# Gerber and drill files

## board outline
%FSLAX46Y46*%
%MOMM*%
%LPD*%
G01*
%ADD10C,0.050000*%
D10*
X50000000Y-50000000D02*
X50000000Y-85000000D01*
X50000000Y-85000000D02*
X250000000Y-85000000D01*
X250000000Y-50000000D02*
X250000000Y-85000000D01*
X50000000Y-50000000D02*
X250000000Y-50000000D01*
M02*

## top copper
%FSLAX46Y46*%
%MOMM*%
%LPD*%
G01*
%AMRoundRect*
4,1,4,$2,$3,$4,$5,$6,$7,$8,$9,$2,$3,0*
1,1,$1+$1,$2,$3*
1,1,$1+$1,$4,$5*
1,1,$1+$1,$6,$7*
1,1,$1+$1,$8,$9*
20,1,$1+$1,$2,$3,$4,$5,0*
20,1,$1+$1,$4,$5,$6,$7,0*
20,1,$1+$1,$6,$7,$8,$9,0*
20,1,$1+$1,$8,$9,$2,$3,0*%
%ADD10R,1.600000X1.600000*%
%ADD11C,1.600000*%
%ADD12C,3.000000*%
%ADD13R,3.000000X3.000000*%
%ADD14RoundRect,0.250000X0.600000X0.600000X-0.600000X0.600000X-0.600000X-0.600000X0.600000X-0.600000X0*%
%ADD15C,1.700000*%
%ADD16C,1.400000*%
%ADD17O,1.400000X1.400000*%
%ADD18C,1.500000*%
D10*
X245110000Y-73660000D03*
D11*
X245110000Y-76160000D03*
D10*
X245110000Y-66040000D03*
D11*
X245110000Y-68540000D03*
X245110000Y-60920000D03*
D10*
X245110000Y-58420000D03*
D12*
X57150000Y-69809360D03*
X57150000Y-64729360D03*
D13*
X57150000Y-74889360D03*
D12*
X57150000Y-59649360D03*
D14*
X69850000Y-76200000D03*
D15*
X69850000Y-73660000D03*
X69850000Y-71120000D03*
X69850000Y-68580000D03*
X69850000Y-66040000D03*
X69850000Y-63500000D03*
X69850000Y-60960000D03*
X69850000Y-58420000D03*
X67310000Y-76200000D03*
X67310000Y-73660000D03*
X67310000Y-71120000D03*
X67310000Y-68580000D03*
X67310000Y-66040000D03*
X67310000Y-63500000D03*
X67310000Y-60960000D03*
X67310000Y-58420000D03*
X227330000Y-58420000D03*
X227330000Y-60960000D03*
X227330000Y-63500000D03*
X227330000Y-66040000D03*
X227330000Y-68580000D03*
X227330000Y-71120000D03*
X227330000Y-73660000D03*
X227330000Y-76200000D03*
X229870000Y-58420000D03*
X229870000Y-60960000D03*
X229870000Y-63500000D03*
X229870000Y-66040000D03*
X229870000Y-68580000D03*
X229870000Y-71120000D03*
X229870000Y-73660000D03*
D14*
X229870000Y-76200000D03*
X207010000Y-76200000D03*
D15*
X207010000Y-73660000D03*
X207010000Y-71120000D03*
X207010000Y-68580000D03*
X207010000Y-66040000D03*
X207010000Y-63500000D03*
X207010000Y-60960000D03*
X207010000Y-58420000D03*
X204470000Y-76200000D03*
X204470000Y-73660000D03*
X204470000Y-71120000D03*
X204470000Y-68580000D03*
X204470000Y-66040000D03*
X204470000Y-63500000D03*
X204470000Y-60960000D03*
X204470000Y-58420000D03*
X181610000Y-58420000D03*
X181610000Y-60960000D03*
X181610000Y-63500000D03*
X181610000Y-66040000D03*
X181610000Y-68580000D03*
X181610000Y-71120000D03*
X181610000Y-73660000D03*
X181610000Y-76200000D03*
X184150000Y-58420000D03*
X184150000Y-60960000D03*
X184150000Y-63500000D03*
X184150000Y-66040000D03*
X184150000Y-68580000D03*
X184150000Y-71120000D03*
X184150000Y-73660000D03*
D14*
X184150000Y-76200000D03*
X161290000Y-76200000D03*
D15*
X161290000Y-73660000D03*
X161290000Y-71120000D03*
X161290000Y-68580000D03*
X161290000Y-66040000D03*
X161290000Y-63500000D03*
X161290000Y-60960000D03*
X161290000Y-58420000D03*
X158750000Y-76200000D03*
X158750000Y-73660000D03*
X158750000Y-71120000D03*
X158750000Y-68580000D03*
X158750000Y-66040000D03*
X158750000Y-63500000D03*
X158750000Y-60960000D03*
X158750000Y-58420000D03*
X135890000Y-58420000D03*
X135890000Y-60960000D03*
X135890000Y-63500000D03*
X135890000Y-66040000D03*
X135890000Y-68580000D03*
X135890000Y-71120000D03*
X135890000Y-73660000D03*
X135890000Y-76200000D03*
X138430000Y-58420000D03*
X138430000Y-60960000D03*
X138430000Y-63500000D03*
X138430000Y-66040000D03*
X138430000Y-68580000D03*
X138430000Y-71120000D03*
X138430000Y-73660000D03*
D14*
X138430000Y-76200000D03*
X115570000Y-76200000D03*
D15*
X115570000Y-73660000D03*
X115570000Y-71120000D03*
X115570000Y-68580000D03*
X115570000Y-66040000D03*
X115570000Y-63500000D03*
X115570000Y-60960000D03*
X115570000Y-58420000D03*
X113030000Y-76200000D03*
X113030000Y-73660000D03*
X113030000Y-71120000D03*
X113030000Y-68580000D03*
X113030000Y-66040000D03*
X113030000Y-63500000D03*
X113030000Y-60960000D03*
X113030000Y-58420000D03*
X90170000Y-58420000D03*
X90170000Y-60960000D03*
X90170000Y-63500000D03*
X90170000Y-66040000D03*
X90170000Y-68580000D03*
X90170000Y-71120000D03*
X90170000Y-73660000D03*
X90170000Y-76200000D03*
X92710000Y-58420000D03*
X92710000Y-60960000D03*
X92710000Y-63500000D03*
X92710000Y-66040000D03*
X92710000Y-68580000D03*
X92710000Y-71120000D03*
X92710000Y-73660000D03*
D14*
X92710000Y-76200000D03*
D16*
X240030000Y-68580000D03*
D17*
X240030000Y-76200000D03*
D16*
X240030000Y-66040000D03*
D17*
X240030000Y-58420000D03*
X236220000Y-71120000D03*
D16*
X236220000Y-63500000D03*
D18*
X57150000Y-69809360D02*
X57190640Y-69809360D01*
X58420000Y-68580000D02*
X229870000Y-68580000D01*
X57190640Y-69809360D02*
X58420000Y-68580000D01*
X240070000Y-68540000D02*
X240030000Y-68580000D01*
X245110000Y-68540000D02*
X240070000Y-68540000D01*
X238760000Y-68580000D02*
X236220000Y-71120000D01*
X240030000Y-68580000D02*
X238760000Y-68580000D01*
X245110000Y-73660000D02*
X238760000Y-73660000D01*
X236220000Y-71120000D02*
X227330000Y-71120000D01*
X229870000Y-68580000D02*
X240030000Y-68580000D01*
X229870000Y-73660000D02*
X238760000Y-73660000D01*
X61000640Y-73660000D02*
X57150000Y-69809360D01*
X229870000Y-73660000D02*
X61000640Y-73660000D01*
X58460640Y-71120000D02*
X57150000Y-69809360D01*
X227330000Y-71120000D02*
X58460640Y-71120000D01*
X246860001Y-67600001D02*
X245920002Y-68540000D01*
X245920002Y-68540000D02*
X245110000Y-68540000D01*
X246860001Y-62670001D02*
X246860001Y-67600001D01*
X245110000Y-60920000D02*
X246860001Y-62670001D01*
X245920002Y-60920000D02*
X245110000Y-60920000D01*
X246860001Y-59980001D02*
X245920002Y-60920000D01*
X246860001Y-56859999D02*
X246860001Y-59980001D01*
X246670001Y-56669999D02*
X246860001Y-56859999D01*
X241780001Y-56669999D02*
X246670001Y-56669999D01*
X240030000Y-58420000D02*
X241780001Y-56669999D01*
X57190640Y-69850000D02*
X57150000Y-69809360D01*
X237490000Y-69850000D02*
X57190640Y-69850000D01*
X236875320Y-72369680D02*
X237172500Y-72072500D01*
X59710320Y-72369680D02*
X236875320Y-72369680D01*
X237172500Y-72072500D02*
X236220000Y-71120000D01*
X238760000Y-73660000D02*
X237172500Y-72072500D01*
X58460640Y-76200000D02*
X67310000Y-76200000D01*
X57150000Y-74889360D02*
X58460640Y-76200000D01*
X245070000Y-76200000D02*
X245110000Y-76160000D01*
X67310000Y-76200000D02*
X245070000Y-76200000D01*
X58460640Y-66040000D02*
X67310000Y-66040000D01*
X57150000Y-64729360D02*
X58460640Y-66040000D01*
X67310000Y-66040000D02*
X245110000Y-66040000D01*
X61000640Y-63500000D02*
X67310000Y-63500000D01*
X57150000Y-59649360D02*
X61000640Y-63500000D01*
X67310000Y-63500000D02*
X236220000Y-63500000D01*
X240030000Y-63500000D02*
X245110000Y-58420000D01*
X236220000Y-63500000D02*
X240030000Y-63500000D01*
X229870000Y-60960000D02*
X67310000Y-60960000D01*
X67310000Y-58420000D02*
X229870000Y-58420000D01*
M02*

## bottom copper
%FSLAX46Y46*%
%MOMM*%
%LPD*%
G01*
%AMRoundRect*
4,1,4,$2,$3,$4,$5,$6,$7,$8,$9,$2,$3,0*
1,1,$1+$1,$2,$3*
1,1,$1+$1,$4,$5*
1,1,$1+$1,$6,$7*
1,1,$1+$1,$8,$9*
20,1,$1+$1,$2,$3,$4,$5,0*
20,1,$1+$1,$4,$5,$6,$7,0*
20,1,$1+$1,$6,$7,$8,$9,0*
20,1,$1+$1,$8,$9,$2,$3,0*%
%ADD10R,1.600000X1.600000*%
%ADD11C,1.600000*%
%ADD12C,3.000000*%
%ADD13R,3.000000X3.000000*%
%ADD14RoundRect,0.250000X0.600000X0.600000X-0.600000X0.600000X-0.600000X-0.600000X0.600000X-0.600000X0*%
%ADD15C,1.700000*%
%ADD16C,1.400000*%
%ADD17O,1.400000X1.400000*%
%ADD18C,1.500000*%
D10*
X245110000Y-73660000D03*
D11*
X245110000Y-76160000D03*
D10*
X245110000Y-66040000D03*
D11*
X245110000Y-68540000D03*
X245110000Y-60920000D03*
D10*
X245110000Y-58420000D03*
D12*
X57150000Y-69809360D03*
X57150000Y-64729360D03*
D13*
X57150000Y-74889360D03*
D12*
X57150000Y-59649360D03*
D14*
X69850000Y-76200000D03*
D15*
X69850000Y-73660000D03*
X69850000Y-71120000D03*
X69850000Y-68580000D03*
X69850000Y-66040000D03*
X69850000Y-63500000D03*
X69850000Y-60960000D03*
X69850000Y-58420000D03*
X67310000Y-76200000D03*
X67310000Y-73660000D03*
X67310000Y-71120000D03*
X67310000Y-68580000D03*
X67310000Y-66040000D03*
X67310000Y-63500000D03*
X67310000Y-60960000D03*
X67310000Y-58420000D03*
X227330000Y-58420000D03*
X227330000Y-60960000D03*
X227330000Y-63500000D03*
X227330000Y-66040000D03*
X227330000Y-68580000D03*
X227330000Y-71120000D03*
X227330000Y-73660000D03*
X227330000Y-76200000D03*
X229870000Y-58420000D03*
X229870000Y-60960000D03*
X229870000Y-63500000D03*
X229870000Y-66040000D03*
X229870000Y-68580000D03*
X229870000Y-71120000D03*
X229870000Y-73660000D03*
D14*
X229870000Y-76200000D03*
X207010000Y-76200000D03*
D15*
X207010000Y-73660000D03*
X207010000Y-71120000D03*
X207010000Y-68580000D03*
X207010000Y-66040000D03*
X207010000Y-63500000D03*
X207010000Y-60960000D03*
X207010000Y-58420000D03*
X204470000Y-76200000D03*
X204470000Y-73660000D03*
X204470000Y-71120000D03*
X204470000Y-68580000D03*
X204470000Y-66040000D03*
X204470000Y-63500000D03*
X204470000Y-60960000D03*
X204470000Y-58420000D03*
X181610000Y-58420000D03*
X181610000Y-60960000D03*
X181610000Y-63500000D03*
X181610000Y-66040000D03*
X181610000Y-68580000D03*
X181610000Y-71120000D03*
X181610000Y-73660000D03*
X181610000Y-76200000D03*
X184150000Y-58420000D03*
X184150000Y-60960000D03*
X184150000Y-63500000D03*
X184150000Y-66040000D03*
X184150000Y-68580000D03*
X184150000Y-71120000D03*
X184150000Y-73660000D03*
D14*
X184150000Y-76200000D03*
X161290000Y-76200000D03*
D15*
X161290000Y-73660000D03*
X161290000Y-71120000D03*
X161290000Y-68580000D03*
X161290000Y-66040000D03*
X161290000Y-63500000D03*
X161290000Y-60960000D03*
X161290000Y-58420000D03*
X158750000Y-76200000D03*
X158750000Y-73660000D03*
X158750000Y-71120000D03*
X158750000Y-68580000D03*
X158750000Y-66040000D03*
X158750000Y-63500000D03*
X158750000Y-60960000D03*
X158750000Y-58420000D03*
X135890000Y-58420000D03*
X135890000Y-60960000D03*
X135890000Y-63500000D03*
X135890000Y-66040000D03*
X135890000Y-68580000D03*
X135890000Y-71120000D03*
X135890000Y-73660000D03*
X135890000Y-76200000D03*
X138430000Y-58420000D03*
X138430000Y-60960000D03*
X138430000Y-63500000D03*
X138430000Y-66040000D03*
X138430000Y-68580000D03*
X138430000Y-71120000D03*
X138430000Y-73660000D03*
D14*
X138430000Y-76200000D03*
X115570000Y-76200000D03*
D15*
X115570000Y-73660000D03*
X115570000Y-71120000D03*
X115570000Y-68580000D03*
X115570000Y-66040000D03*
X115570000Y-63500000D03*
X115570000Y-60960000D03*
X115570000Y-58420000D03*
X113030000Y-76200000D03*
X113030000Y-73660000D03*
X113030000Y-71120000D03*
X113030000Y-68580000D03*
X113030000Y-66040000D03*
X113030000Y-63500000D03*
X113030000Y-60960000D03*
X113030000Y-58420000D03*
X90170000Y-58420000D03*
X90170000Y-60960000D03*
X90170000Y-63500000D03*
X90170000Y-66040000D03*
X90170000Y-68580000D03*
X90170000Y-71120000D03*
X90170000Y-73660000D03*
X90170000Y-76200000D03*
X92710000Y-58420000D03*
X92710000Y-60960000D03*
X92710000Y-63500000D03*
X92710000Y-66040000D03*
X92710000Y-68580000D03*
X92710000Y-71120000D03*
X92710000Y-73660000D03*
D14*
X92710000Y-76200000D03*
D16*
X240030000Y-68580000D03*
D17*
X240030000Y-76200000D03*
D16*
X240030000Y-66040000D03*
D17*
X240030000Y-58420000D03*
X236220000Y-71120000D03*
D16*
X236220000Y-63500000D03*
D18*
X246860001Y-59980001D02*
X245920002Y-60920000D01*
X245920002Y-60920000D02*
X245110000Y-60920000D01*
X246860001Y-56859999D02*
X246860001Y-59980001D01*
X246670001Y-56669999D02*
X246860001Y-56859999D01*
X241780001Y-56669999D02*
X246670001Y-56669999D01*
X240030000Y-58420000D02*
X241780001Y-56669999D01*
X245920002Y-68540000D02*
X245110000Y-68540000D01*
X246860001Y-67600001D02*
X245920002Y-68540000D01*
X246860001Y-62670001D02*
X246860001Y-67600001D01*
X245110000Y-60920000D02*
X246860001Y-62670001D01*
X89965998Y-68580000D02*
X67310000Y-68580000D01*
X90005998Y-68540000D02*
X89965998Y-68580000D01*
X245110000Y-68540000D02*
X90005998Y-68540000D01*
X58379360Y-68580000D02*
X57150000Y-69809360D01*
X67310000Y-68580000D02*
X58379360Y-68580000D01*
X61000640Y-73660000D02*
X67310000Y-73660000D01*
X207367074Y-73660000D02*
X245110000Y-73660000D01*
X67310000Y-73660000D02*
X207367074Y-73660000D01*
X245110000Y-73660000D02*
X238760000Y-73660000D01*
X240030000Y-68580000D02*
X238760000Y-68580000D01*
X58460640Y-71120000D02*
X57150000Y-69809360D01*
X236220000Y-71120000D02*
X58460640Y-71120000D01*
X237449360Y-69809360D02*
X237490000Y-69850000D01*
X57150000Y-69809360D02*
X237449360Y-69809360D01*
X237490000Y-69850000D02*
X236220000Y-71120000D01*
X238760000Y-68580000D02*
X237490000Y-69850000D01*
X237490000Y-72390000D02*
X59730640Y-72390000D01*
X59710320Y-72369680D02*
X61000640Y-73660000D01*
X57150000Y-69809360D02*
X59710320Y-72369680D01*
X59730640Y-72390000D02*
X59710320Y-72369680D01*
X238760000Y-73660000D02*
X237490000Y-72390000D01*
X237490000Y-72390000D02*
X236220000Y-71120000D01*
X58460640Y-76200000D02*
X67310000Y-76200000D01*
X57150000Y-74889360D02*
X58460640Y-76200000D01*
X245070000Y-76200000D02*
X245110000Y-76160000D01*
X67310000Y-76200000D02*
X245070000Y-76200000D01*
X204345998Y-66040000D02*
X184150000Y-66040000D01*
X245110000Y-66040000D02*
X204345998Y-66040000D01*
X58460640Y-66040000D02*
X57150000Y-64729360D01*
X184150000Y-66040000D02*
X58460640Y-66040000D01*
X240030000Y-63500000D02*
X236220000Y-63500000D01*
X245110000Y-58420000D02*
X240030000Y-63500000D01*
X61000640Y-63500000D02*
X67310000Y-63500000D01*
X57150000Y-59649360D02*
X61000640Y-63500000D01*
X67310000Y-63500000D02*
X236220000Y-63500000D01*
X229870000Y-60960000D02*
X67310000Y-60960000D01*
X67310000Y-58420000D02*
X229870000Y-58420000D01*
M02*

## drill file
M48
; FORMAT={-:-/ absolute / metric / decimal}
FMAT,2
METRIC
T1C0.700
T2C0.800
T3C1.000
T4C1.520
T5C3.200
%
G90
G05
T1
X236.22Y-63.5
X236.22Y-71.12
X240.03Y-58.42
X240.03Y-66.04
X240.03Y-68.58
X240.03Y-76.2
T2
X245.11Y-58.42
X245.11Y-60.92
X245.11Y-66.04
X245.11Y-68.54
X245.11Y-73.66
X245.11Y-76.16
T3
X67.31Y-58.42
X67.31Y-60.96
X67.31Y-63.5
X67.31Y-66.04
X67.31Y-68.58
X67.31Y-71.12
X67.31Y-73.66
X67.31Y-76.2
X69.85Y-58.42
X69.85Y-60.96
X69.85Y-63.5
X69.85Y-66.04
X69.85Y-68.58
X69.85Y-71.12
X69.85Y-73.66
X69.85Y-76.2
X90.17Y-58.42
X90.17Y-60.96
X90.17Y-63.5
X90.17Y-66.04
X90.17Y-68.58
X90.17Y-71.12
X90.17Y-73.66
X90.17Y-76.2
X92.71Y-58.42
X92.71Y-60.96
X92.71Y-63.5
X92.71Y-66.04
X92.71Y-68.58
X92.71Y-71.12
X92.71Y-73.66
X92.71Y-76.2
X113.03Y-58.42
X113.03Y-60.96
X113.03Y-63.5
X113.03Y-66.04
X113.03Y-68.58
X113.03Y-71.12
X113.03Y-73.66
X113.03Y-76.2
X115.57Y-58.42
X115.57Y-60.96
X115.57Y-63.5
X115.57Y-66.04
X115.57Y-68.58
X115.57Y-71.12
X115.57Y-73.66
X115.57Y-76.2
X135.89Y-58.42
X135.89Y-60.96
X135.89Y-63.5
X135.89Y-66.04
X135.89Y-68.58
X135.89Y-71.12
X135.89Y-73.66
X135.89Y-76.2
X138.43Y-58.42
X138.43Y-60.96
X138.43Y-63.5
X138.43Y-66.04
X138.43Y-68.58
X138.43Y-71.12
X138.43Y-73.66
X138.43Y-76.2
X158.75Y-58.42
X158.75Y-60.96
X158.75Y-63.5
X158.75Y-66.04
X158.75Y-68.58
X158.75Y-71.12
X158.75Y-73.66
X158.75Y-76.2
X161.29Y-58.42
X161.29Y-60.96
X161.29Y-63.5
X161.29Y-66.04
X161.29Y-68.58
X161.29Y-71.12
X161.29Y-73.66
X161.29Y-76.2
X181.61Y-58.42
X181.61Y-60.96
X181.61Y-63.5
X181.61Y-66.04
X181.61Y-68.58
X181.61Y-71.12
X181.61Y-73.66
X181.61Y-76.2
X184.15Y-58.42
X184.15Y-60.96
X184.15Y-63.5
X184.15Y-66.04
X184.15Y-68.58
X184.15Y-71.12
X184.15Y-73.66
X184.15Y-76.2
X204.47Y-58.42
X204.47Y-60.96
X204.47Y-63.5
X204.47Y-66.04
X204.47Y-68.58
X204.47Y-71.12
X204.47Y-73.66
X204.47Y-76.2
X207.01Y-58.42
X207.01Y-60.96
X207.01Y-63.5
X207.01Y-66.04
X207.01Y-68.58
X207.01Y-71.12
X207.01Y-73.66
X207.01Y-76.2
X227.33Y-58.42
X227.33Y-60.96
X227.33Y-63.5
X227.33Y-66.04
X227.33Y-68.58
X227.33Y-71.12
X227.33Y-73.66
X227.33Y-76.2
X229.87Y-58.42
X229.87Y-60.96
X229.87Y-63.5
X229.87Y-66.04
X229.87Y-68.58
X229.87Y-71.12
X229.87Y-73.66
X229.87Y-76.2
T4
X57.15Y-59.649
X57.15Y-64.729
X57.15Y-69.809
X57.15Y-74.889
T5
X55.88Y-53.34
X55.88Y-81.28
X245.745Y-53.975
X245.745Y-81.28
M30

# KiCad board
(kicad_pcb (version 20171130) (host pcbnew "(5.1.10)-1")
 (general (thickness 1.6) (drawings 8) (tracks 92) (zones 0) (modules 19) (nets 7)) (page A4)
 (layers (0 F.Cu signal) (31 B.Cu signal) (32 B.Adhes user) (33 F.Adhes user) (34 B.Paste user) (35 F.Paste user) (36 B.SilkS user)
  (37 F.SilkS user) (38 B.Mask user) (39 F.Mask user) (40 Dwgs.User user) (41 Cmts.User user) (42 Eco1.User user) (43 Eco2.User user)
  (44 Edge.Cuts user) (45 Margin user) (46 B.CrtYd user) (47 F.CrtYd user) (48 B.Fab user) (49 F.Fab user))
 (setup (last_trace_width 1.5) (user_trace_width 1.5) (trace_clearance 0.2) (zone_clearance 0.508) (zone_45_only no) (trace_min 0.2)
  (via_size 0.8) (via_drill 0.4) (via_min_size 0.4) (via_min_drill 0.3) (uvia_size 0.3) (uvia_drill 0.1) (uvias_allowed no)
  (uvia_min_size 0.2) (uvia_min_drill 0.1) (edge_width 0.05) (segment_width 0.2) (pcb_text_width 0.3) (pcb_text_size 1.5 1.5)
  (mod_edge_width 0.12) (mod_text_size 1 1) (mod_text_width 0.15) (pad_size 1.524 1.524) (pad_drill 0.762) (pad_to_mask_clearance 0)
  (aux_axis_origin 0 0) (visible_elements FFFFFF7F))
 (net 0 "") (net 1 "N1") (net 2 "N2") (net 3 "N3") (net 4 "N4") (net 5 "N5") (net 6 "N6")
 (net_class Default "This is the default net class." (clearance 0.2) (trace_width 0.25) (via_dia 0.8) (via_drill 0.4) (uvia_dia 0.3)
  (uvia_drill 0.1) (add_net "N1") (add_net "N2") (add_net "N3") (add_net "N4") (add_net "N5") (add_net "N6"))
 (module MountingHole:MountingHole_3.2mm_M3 (layer F.Cu) (at 245.745 81.28)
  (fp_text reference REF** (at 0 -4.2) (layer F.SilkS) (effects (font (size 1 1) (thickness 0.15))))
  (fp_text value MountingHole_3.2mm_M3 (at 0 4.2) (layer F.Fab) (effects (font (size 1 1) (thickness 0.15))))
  (pad 1 np_thru_hole circle (at 0 0) (size 3.2 3.2) (drill 3.2) (layers *.Cu *.Mask)))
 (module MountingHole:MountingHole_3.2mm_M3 (layer F.Cu) (at 245.745 53.975)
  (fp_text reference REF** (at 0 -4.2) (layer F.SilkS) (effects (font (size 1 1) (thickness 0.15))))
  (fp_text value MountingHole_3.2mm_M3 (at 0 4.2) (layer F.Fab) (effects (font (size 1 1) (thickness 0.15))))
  (pad 1 np_thru_hole circle (at 0 0) (size 3.2 3.2) (drill 3.2) (layers *.Cu *.Mask)))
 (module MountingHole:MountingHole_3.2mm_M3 (layer F.Cu) (at 55.88 53.34)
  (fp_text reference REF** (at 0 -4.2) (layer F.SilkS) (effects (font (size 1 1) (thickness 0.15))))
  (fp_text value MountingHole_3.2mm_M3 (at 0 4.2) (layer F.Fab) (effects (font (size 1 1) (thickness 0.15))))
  (pad 1 np_thru_hole circle (at 0 0) (size 3.2 3.2) (drill 3.2) (layers *.Cu *.Mask)))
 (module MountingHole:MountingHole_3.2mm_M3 (layer F.Cu) (at 55.88 81.28)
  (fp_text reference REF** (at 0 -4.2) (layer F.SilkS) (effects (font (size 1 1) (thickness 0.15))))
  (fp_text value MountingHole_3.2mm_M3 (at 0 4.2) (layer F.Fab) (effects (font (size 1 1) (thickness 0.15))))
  (pad 1 np_thru_hole circle (at 0 0) (size 3.2 3.2) (drill 3.2) (layers *.Cu *.Mask)))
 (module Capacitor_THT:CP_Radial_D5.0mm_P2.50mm (layer F.Cu) (at 245.11 73.66 270)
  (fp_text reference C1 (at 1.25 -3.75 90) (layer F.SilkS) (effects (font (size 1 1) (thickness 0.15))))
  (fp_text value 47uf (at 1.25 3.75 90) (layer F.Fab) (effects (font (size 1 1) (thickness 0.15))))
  (pad 1 thru_hole rect (at 0 0 270) (size 1.6 1.6) (drill 0.8) (layers *.Cu *.Mask) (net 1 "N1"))
  (pad 2 thru_hole circle (at 2.5 0 270) (size 1.6 1.6) (drill 0.8) (layers *.Cu *.Mask) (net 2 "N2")))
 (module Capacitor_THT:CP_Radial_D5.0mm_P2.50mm (layer F.Cu) (at 245.11 66.04 270)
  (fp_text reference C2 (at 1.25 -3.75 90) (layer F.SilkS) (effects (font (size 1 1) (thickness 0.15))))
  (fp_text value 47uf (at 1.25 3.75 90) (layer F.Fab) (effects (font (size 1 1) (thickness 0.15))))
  (pad 1 thru_hole rect (at 0 0 270) (size 1.6 1.6) (drill 0.8) (layers *.Cu *.Mask) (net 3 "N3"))
  (pad 2 thru_hole circle (at 2.5 0 270) (size 1.6 1.6) (drill 0.8) (layers *.Cu *.Mask) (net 1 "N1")))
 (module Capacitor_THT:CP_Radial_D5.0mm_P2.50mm (layer F.Cu) (at 245.11 58.42 270)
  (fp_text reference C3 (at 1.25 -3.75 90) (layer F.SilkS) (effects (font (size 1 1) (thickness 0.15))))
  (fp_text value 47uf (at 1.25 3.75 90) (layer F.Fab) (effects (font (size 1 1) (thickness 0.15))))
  (pad 2 thru_hole circle (at 2.5 0 270) (size 1.6 1.6) (drill 0.8) (layers *.Cu *.Mask) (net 1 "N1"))
  (pad 1 thru_hole rect (at 0 0 270) (size 1.6 1.6) (drill 0.8) (layers *.Cu *.Mask) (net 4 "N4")))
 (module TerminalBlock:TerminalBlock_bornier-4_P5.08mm (layer F.Cu) (at 57.15 74.88936 90)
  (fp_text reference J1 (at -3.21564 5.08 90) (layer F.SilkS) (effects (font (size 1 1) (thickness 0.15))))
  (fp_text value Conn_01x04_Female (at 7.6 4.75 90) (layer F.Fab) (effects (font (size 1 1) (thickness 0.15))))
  (pad 2 thru_hole circle (at 5.08 0 90) (size 3 3) (drill 1.52) (layers *.Cu *.Mask) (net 1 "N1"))
  (pad 3 thru_hole circle (at 10.16 0 90) (size 3 3) (drill 1.52) (layers *.Cu *.Mask) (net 3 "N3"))
  (pad 1 thru_hole rect (at 0 0 90) (size 3 3) (drill 1.52) (layers *.Cu *.Mask) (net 2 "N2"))
  (pad 4 thru_hole circle (at 15.24 0 90) (size 3 3) (drill 1.52) (layers *.Cu *.Mask) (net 4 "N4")))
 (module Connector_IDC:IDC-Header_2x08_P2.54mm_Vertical (layer F.Cu) (at 69.85 76.2 180)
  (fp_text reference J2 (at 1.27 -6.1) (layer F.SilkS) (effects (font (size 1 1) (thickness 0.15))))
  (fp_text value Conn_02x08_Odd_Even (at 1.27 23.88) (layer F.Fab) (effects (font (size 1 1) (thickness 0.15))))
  (pad 1 thru_hole roundrect (at 0 0 180) (size 1.7 1.7) (drill 1) (layers *.Cu *.Mask) (roundrect_rratio 0.1470588235294118) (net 2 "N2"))
  (pad 3 thru_hole circle (at 0 2.54 180) (size 1.7 1.7) (drill 1) (layers *.Cu *.Mask) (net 1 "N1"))
  (pad 5 thru_hole circle (at 0 5.08 180) (size 1.7 1.7) (drill 1) (layers *.Cu *.Mask) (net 1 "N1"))
  (pad 7 thru_hole circle (at 0 7.62 180) (size 1.7 1.7) (drill 1) (layers *.Cu *.Mask) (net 1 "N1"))
  (pad 9 thru_hole circle (at 0 10.16 180) (size 1.7 1.7) (drill 1) (layers *.Cu *.Mask) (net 3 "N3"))
  (pad 11 thru_hole circle (at 0 12.7 180) (size 1.7 1.7) (drill 1) (layers *.Cu *.Mask) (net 4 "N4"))
  (pad 13 thru_hole circle (at 0 15.24 180) (size 1.7 1.7) (drill 1) (layers *.Cu *.Mask) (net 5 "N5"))
  (pad 15 thru_hole circle (at 0 17.78 180) (size 1.7 1.7) (drill 1) (layers *.Cu *.Mask) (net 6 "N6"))
  (pad 2 thru_hole circle (at 2.54 0 180) (size 1.7 1.7) (drill 1) (layers *.Cu *.Mask) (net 2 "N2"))
  (pad 4 thru_hole circle (at 2.54 2.54 180) (size 1.7 1.7) (drill 1) (layers *.Cu *.Mask) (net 1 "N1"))
  (pad 6 thru_hole circle (at 2.54 5.08 180) (size 1.7 1.7) (drill 1) (layers *.Cu *.Mask) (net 1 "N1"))
  (pad 8 thru_hole circle (at 2.54 7.62 180) (size 1.7 1.7) (drill 1) (layers *.Cu *.Mask) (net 1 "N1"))
  (pad 10 thru_hole circle (at 2.54 10.16 180) (size 1.7 1.7) (drill 1) (layers *.Cu *.Mask) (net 3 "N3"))
  (pad 12 thru_hole circle (at 2.54 12.7 180) (size 1.7 1.7) (drill 1) (layers *.Cu *.Mask) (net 4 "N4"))
  (pad 14 thru_hole circle (at 2.54 15.24 180) (size 1.7 1.7) (drill 1) (layers *.Cu *.Mask) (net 5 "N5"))
  (pad 16 thru_hole circle (at 2.54 17.78 180) (size 1.7 1.7) (drill 1) (layers *.Cu *.Mask) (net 6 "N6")))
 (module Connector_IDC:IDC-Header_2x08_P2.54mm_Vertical (layer F.Cu) (at 229.87 76.2 180)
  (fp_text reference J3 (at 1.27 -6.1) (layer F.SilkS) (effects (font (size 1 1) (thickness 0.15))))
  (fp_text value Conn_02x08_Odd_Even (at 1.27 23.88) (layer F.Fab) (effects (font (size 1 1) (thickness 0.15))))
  (pad 16 thru_hole circle (at 2.54 17.78 180) (size 1.7 1.7) (drill 1) (layers *.Cu *.Mask) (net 6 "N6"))
  (pad 14 thru_hole circle (at 2.54 15.24 180) (size 1.7 1.7) (drill 1) (layers *.Cu *.Mask) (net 5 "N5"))
  (pad 12 thru_hole circle (at 2.54 12.7 180) (size 1.7 1.7) (drill 1) (layers *.Cu *.Mask) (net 4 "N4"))
  (pad 10 thru_hole circle (at 2.54 10.16 180) (size 1.7 1.7) (drill 1) (layers *.Cu *.Mask) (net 3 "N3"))
  (pad 8 thru_hole circle (at 2.54 7.62 180) (size 1.7 1.7) (drill 1) (layers *.Cu *.Mask) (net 1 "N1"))
  (pad 6 thru_hole circle (at 2.54 5.08 180) (size 1.7 1.7) (drill 1) (layers *.Cu *.Mask) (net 1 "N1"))
  (pad 4 thru_hole circle (at 2.54 2.54 180) (size 1.7 1.7) (drill 1) (layers *.Cu *.Mask) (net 1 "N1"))
  (pad 2 thru_hole circle (at 2.54 0 180) (size 1.7 1.7) (drill 1) (layers *.Cu *.Mask) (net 2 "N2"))
  (pad 15 thru_hole circle (at 0 17.78 180) (size 1.7 1.7) (drill 1) (layers *.Cu *.Mask) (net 6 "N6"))
  (pad 13 thru_hole circle (at 0 15.24 180) (size 1.7 1.7) (drill 1) (layers *.Cu *.Mask) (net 5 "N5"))
  (pad 11 thru_hole circle (at 0 12.7 180) (size 1.7 1.7) (drill 1) (layers *.Cu *.Mask) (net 4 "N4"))
  (pad 9 thru_hole circle (at 0 10.16 180) (size 1.7 1.7) (drill 1) (layers *.Cu *.Mask) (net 3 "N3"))
  (pad 7 thru_hole circle (at 0 7.62 180) (size 1.7 1.7) (drill 1) (layers *.Cu *.Mask) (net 1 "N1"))
  (pad 5 thru_hole circle (at 0 5.08 180) (size 1.7 1.7) (drill 1) (layers *.Cu *.Mask) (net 1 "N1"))
  (pad 3 thru_hole circle (at 0 2.54 180) (size 1.7 1.7) (drill 1) (layers *.Cu *.Mask) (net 1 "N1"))
  (pad 1 thru_hole roundrect (at 0 0 180) (size 1.7 1.7) (drill 1) (layers *.Cu *.Mask) (roundrect_rratio 0.1470588235294118) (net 2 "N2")))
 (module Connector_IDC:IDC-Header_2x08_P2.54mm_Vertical (layer F.Cu) (at 207.01 76.2 180)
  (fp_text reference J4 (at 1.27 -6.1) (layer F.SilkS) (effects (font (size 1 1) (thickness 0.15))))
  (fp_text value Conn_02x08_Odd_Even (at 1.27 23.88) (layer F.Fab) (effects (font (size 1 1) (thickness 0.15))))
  (pad 1 thru_hole roundrect (at 0 0 180) (size 1.7 1.7) (drill 1) (layers *.Cu *.Mask) (roundrect_rratio 0.1470588235294118) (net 2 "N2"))
  (pad 3 thru_hole circle (at 0 2.54 180) (size 1.7 1.7) (drill 1) (layers *.Cu *.Mask) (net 1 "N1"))
  (pad 5 thru_hole circle (at 0 5.08 180) (size 1.7 1.7) (drill 1) (layers *.Cu *.Mask) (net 1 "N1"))
  (pad 7 thru_hole circle (at 0 7.62 180) (size 1.7 1.7) (drill 1) (layers *.Cu *.Mask) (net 1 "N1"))
  (pad 9 thru_hole circle (at 0 10.16 180) (size 1.7 1.7) (drill 1) (layers *.Cu *.Mask) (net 3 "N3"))
  (pad 11 thru_hole circle (at 0 12.7 180) (size 1.7 1.7) (drill 1) (layers *.Cu *.Mask) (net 4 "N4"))
  (pad 13 thru_hole circle (at 0 15.24 180) (size 1.7 1.7) (drill 1) (layers *.Cu *.Mask) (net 5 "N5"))
  (pad 15 thru_hole circle (at 0 17.78 180) (size 1.7 1.7) (drill 1) (layers *.Cu *.Mask) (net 6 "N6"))
  (pad 2 thru_hole circle (at 2.54 0 180) (size 1.7 1.7) (drill 1) (layers *.Cu *.Mask) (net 2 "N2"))
  (pad 4 thru_hole circle (at 2.54 2.54 180) (size 1.7 1.7) (drill 1) (layers *.Cu *.Mask) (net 1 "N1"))
  (pad 6 thru_hole circle (at 2.54 5.08 180) (size 1.7 1.7) (drill 1) (layers *.Cu *.Mask) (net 1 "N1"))
  (pad 8 thru_hole circle (at 2.54 7.62 180) (size 1.7 1.7) (drill 1) (layers *.Cu *.Mask) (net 1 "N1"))
  (pad 10 thru_hole circle (at 2.54 10.16 180) (size 1.7 1.7) (drill 1) (layers *.Cu *.Mask) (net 3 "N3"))
  (pad 12 thru_hole circle (at 2.54 12.7 180) (size 1.7 1.7) (drill 1) (layers *.Cu *.Mask) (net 4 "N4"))
  (pad 14 thru_hole circle (at 2.54 15.24 180) (size 1.7 1.7) (drill 1) (layers *.Cu *.Mask) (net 5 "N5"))
  (pad 16 thru_hole circle (at 2.54 17.78 180) (size 1.7 1.7) (drill 1) (layers *.Cu *.Mask) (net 6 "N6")))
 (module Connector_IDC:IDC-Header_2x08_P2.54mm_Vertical (layer F.Cu) (at 184.15 76.2 180)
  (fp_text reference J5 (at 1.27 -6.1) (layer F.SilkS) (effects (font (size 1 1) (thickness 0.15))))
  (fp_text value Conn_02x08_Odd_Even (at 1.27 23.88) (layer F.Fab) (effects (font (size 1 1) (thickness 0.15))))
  (pad 16 thru_hole circle (at 2.54 17.78 180) (size 1.7 1.7) (drill 1) (layers *.Cu *.Mask) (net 6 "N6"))
  (pad 14 thru_hole circle (at 2.54 15.24 180) (size 1.7 1.7) (drill 1) (layers *.Cu *.Mask) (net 5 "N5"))
  (pad 12 thru_hole circle (at 2.54 12.7 180) (size 1.7 1.7) (drill 1) (layers *.Cu *.Mask) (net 4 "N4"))
  (pad 10 thru_hole circle (at 2.54 10.16 180) (size 1.7 1.7) (drill 1) (layers *.Cu *.Mask) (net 3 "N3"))
  (pad 8 thru_hole circle (at 2.54 7.62 180) (size 1.7 1.7) (drill 1) (layers *.Cu *.Mask) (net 1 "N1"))
  (pad 6 thru_hole circle (at 2.54 5.08 180) (size 1.7 1.7) (drill 1) (layers *.Cu *.Mask) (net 1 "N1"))
  (pad 4 thru_hole circle (at 2.54 2.54 180) (size 1.7 1.7) (drill 1) (layers *.Cu *.Mask) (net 1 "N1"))
  (pad 2 thru_hole circle (at 2.54 0 180) (size 1.7 1.7) (drill 1) (layers *.Cu *.Mask) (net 2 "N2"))
  (pad 15 thru_hole circle (at 0 17.78 180) (size 1.7 1.7) (drill 1) (layers *.Cu *.Mask) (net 6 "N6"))
  (pad 13 thru_hole circle (at 0 15.24 180) (size 1.7 1.7) (drill 1) (layers *.Cu *.Mask) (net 5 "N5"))
  (pad 11 thru_hole circle (at 0 12.7 180) (size 1.7 1.7) (drill 1) (layers *.Cu *.Mask) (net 4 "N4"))
  (pad 9 thru_hole circle (at 0 10.16 180) (size 1.7 1.7) (drill 1) (layers *.Cu *.Mask) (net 3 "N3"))
  (pad 7 thru_hole circle (at 0 7.62 180) (size 1.7 1.7) (drill 1) (layers *.Cu *.Mask) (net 1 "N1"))
  (pad 5 thru_hole circle (at 0 5.08 180) (size 1.7 1.7) (drill 1) (layers *.Cu *.Mask) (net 1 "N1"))
  (pad 3 thru_hole circle (at 0 2.54 180) (size 1.7 1.7) (drill 1) (layers *.Cu *.Mask) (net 1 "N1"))
  (pad 1 thru_hole roundrect (at 0 0 180) (size 1.7 1.7) (drill 1) (layers *.Cu *.Mask) (roundrect_rratio 0.1470588235294118) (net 2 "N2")))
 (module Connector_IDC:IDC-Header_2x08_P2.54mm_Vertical (layer F.Cu) (at 161.29 76.2 180)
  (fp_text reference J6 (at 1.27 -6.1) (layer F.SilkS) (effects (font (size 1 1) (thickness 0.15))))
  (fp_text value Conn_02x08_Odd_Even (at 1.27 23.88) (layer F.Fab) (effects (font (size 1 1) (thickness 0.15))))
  (pad 1 thru_hole roundrect (at 0 0 180) (size 1.7 1.7) (drill 1) (layers *.Cu *.Mask) (roundrect_rratio 0.1470588235294118) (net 2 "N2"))
  (pad 3 thru_hole circle (at 0 2.54 180) (size 1.7 1.7) (drill 1) (layers *.Cu *.Mask) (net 1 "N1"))
  (pad 5 thru_hole circle (at 0 5.08 180) (size 1.7 1.7) (drill 1) (layers *.Cu *.Mask) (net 1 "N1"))
  (pad 7 thru_hole circle (at 0 7.62 180) (size 1.7 1.7) (drill 1) (layers *.Cu *.Mask) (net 1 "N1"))
  (pad 9 thru_hole circle (at 0 10.16 180) (size 1.7 1.7) (drill 1) (layers *.Cu *.Mask) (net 3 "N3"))
  (pad 11 thru_hole circle (at 0 12.7 180) (size 1.7 1.7) (drill 1) (layers *.Cu *.Mask) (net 4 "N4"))
  (pad 13 thru_hole circle (at 0 15.24 180) (size 1.7 1.7) (drill 1) (layers *.Cu *.Mask) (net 5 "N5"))
  (pad 15 thru_hole circle (at 0 17.78 180) (size 1.7 1.7) (drill 1) (layers *.Cu *.Mask) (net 6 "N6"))
  (pad 2 thru_hole circle (at 2.54 0 180) (size 1.7 1.7) (drill 1) (layers *.Cu *.Mask) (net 2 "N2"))
  (pad 4 thru_hole circle (at 2.54 2.54 180) (size 1.7 1.7) (drill 1) (layers *.Cu *.Mask) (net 1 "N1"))
  (pad 6 thru_hole circle (at 2.54 5.08 180) (size 1.7 1.7) (drill 1) (layers *.Cu *.Mask) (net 1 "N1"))
  (pad 8 thru_hole circle (at 2.54 7.62 180) (size 1.7 1.7) (drill 1) (layers *.Cu *.Mask) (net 1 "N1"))
  (pad 10 thru_hole circle (at 2.54 10.16 180) (size 1.7 1.7) (drill 1) (layers *.Cu *.Mask) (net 3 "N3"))
  (pad 12 thru_hole circle (at 2.54 12.7 180) (size 1.7 1.7) (drill 1) (layers *.Cu *.Mask) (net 4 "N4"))
  (pad 14 thru_hole circle (at 2.54 15.24 180) (size 1.7 1.7) (drill 1) (layers *.Cu *.Mask) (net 5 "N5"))
  (pad 16 thru_hole circle (at 2.54 17.78 180) (size 1.7 1.7) (drill 1) (layers *.Cu *.Mask) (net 6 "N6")))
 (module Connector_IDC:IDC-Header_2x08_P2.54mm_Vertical (layer F.Cu) (at 138.43 76.2 180)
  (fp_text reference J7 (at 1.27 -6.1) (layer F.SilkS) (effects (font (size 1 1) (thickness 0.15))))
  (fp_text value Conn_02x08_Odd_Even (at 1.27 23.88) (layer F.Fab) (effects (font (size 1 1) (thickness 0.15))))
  (pad 16 thru_hole circle (at 2.54 17.78 180) (size 1.7 1.7) (drill 1) (layers *.Cu *.Mask) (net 6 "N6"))
  (pad 14 thru_hole circle (at 2.54 15.24 180) (size 1.7 1.7) (drill 1) (layers *.Cu *.Mask) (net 5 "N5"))
  (pad 12 thru_hole circle (at 2.54 12.7 180) (size 1.7 1.7) (drill 1) (layers *.Cu *.Mask) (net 4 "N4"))
  (pad 10 thru_hole circle (at 2.54 10.16 180) (size 1.7 1.7) (drill 1) (layers *.Cu *.Mask) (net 3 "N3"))
  (pad 8 thru_hole circle (at 2.54 7.62 180) (size 1.7 1.7) (drill 1) (layers *.Cu *.Mask) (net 1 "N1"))
  (pad 6 thru_hole circle (at 2.54 5.08 180) (size 1.7 1.7) (drill 1) (layers *.Cu *.Mask) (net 1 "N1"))
  (pad 4 thru_hole circle (at 2.54 2.54 180) (size 1.7 1.7) (drill 1) (layers *.Cu *.Mask) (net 1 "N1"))
  (pad 2 thru_hole circle (at 2.54 0 180) (size 1.7 1.7) (drill 1) (layers *.Cu *.Mask) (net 2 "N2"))
  (pad 15 thru_hole circle (at 0 17.78 180) (size 1.7 1.7) (drill 1) (layers *.Cu *.Mask) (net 6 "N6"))
  (pad 13 thru_hole circle (at 0 15.24 180) (size 1.7 1.7) (drill 1) (layers *.Cu *.Mask) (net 5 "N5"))
  (pad 11 thru_hole circle (at 0 12.7 180) (size 1.7 1.7) (drill 1) (layers *.Cu *.Mask) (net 4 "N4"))
  (pad 9 thru_hole circle (at 0 10.16 180) (size 1.7 1.7) (drill 1) (layers *.Cu *.Mask) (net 3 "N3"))
  (pad 7 thru_hole circle (at 0 7.62 180) (size 1.7 1.7) (drill 1) (layers *.Cu *.Mask) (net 1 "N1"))
  (pad 5 thru_hole circle (at 0 5.08 180) (size 1.7 1.7) (drill 1) (layers *.Cu *.Mask) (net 1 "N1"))
  (pad 3 thru_hole circle (at 0 2.54 180) (size 1.7 1.7) (drill 1) (layers *.Cu *.Mask) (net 1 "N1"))
  (pad 1 thru_hole roundrect (at 0 0 180) (size 1.7 1.7) (drill 1) (layers *.Cu *.Mask) (roundrect_rratio 0.1470588235294118) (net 2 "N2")))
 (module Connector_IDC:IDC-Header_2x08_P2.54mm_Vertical (layer F.Cu) (at 115.57 76.2 180)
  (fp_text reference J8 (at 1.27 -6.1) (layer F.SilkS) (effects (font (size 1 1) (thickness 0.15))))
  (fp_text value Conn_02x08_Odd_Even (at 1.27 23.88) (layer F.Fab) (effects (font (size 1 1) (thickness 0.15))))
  (pad 1 thru_hole roundrect (at 0 0 180) (size 1.7 1.7) (drill 1) (layers *.Cu *.Mask) (roundrect_rratio 0.1470588235294118) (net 2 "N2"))
  (pad 3 thru_hole circle (at 0 2.54 180) (size 1.7 1.7) (drill 1) (layers *.Cu *.Mask) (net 1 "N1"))
  (pad 5 thru_hole circle (at 0 5.08 180) (size 1.7 1.7) (drill 1) (layers *.Cu *.Mask) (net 1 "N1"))
  (pad 7 thru_hole circle (at 0 7.62 180) (size 1.7 1.7) (drill 1) (layers *.Cu *.Mask) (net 1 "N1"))
  (pad 9 thru_hole circle (at 0 10.16 180) (size 1.7 1.7) (drill 1) (layers *.Cu *.Mask) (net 3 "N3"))
  (pad 11 thru_hole circle (at 0 12.7 180) (size 1.7 1.7) (drill 1) (layers *.Cu *.Mask) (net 4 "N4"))
  (pad 13 thru_hole circle (at 0 15.24 180) (size 1.7 1.7) (drill 1) (layers *.Cu *.Mask) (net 5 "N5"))
  (pad 15 thru_hole circle (at 0 17.78 180) (size 1.7 1.7) (drill 1) (layers *.Cu *.Mask) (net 6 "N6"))
  (pad 2 thru_hole circle (at 2.54 0 180) (size 1.7 1.7) (drill 1) (layers *.Cu *.Mask) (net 2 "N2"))
  (pad 4 thru_hole circle (at 2.54 2.54 180) (size 1.7 1.7) (drill 1) (layers *.Cu *.Mask) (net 1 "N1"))
  (pad 6 thru_hole circle (at 2.54 5.08 180) (size 1.7 1.7) (drill 1) (layers *.Cu *.Mask) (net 1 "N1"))
  (pad 8 thru_hole circle (at 2.54 7.62 180) (size 1.7 1.7) (drill 1) (layers *.Cu *.Mask) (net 1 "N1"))
  (pad 10 thru_hole circle (at 2.54 10.16 180) (size 1.7 1.7) (drill 1) (layers *.Cu *.Mask) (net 3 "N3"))
  (pad 12 thru_hole circle (at 2.54 12.7 180) (size 1.7 1.7) (drill 1) (layers *.Cu *.Mask) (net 4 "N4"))
  (pad 14 thru_hole circle (at 2.54 15.24 180) (size 1.7 1.7) (drill 1) (layers *.Cu *.Mask) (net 5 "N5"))
  (pad 16 thru_hole circle (at 2.54 17.78 180) (size 1.7 1.7) (drill 1) (layers *.Cu *.Mask) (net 6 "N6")))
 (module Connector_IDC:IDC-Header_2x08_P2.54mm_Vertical (layer F.Cu) (at 92.71 76.2 180)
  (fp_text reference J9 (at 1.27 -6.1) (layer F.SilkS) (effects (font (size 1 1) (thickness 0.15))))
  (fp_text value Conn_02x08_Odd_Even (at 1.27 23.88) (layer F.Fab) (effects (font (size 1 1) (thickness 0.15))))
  (pad 16 thru_hole circle (at 2.54 17.78 180) (size 1.7 1.7) (drill 1) (layers *.Cu *.Mask) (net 6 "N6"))
  (pad 14 thru_hole circle (at 2.54 15.24 180) (size 1.7 1.7) (drill 1) (layers *.Cu *.Mask) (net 5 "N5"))
  (pad 12 thru_hole circle (at 2.54 12.7 180) (size 1.7 1.7) (drill 1) (layers *.Cu *.Mask) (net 4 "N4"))
  (pad 10 thru_hole circle (at 2.54 10.16 180) (size 1.7 1.7) (drill 1) (layers *.Cu *.Mask) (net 3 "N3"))
  (pad 8 thru_hole circle (at 2.54 7.62 180) (size 1.7 1.7) (drill 1) (layers *.Cu *.Mask) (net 1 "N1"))
  (pad 6 thru_hole circle (at 2.54 5.08 180) (size 1.7 1.7) (drill 1) (layers *.Cu *.Mask) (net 1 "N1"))
  (pad 4 thru_hole circle (at 2.54 2.54 180) (size 1.7 1.7) (drill 1) (layers *.Cu *.Mask) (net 1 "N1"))
  (pad 2 thru_hole circle (at 2.54 0 180) (size 1.7 1.7) (drill 1) (layers *.Cu *.Mask) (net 2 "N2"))
  (pad 15 thru_hole circle (at 0 17.78 180) (size 1.7 1.7) (drill 1) (layers *.Cu *.Mask) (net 6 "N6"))
  (pad 13 thru_hole circle (at 0 15.24 180) (size 1.7 1.7) (drill 1) (layers *.Cu *.Mask) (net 5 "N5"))
  (pad 11 thru_hole circle (at 0 12.7 180) (size 1.7 1.7) (drill 1) (layers *.Cu *.Mask) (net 4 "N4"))
  (pad 9 thru_hole circle (at 0 10.16 180) (size 1.7 1.7) (drill 1) (layers *.Cu *.Mask) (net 3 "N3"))
  (pad 7 thru_hole circle (at 0 7.62 180) (size 1.7 1.7) (drill 1) (layers *.Cu *.Mask) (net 1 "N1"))
  (pad 5 thru_hole circle (at 0 5.08 180) (size 1.7 1.7) (drill 1) (layers *.Cu *.Mask) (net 1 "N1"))
  (pad 3 thru_hole circle (at 0 2.54 180) (size 1.7 1.7) (drill 1) (layers *.Cu *.Mask) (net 1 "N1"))
  (pad 1 thru_hole roundrect (at 0 0 180) (size 1.7 1.7) (drill 1) (layers *.Cu *.Mask) (roundrect_rratio 0.1470588235294118) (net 2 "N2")))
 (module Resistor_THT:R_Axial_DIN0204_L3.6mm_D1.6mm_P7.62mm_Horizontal (layer F.Cu) (at 240.03 68.58 270)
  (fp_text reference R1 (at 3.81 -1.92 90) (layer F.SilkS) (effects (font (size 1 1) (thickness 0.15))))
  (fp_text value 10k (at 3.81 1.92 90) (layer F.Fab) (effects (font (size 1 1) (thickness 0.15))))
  (pad 1 thru_hole circle (at 0 0 270) (size 1.4 1.4) (drill 0.7) (layers *.Cu *.Mask) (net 1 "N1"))
  (pad 2 thru_hole oval (at 7.62 0 270) (size 1.4 1.4) (drill 0.7) (layers *.Cu *.Mask) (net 2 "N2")))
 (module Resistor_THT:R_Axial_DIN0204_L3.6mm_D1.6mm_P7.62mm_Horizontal (layer F.Cu) (at 240.03 66.04 90)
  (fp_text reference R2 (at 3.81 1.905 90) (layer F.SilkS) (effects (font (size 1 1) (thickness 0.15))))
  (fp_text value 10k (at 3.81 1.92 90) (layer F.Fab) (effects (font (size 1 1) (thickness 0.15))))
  (pad 1 thru_hole circle (at 0 0 90) (size 1.4 1.4) (drill 0.7) (layers *.Cu *.Mask) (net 3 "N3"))
  (pad 2 thru_hole oval (at 7.62 0 90) (size 1.4 1.4) (drill 0.7) (layers *.Cu *.Mask) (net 1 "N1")))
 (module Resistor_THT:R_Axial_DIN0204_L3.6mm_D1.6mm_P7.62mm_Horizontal (layer F.Cu) (at 236.22 63.5 270)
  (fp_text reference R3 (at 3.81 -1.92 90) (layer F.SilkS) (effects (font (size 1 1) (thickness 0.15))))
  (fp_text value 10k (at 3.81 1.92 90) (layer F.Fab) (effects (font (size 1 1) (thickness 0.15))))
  (pad 2 thru_hole oval (at 7.62 0 270) (size 1.4 1.4) (drill 0.7) (layers *.Cu *.Mask) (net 1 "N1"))
  (pad 1 thru_hole circle (at 0 0 270) (size 1.4 1.4) (drill 0.7) (layers *.Cu *.Mask) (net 4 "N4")))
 (gr_line (start 50 50) (end 50 85) (layer Edge.Cuts) (width 0.05))
 (gr_line (start 50 85) (end 250 85) (layer Edge.Cuts) (width 0.05))
 (gr_line (start 250 50) (end 250 85) (layer Edge.Cuts) (width 0.05))
 (gr_line (start 50 50) (end 250 50) (layer Edge.Cuts) (width 0.05))
 (segment (start 57.15 69.80936) (end 57.19064 69.80936) (width 1.5) (layer F.Cu) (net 1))
 (segment (start 58.42 68.58) (end 229.87 68.58) (width 1.5) (layer F.Cu) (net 1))
 (segment (start 57.19064 69.80936) (end 58.42 68.58) (width 1.5) (layer F.Cu) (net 1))
 (segment (start 240.07 68.54) (end 240.03 68.58) (width 1.5) (layer F.Cu) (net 1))
 (segment (start 245.11 68.54) (end 240.07 68.54) (width 1.5) (layer F.Cu) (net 1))
 (segment (start 238.76 68.58) (end 236.22 71.12) (width 1.5) (layer F.Cu) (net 1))
 (segment (start 240.03 68.58) (end 238.76 68.58) (width 1.5) (layer F.Cu) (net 1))
 (segment (start 245.11 73.66) (end 238.76 73.66) (width 1.5) (layer F.Cu) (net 1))
 (segment (start 236.22 71.12) (end 227.33 71.12) (width 1.5) (layer F.Cu) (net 1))
 (segment (start 229.87 68.58) (end 240.03 68.58) (width 1.5) (layer F.Cu) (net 1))
 (segment (start 229.87 73.66) (end 238.76 73.66) (width 1.5) (layer F.Cu) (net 1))
 (segment (start 61.00064 73.66) (end 57.15 69.80936) (width 1.5) (layer F.Cu) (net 1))
 (segment (start 229.87 73.66) (end 61.00064 73.66) (width 1.5) (layer F.Cu) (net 1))
 (segment (start 58.46064 71.12) (end 57.15 69.80936) (width 1.5) (layer F.Cu) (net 1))
 (segment (start 227.33 71.12) (end 58.46064 71.12) (width 1.5) (layer F.Cu) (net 1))
 (segment (start 246.860001 67.600001) (end 245.920002 68.54) (width 1.5) (layer F.Cu) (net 1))
 (segment (start 245.920002 68.54) (end 245.11 68.54) (width 1.5) (layer F.Cu) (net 1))
 (segment (start 246.860001 62.670001) (end 246.860001 67.600001) (width 1.5) (layer F.Cu) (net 1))
 (segment (start 245.11 60.92) (end 246.860001 62.670001) (width 1.5) (layer F.Cu) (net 1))
 (segment (start 245.920002 60.92) (end 245.11 60.92) (width 1.5) (layer F.Cu) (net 1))
 (segment (start 246.860001 59.980001) (end 245.920002 60.92) (width 1.5) (layer F.Cu) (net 1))
 (segment (start 246.860001 56.859999) (end 246.860001 59.980001) (width 1.5) (layer F.Cu) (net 1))
 (segment (start 246.670001 56.669999) (end 246.860001 56.859999) (width 1.5) (layer F.Cu) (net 1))
 (segment (start 241.780001 56.669999) (end 246.670001 56.669999) (width 1.5) (layer F.Cu) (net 1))
 (segment (start 240.03 58.42) (end 241.780001 56.669999) (width 1.5) (layer F.Cu) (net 1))
 (segment (start 246.860001 59.980001) (end 245.920002 60.92) (width 1.5) (layer B.Cu) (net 1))
 (segment (start 245.920002 60.92) (end 245.11 60.92) (width 1.5) (layer B.Cu) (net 1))
 (segment (start 246.860001 56.859999) (end 246.860001 59.980001) (width 1.5) (layer B.Cu) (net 1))
 (segment (start 246.670001 56.669999) (end 246.860001 56.859999) (width 1.5) (layer B.Cu) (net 1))
 (segment (start 241.780001 56.669999) (end 246.670001 56.669999) (width 1.5) (layer B.Cu) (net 1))
 (segment (start 240.03 58.42) (end 241.780001 56.669999) (width 1.5) (layer B.Cu) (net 1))
 (segment (start 245.920002 68.54) (end 245.11 68.54) (width 1.5) (layer B.Cu) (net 1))
 (segment (start 246.860001 67.600001) (end 245.920002 68.54) (width 1.5) (layer B.Cu) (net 1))
 (segment (start 246.860001 62.670001) (end 246.860001 67.600001) (width 1.5) (layer B.Cu) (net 1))
 (segment (start 245.11 60.92) (end 246.860001 62.670001) (width 1.5) (layer B.Cu) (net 1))
 (segment (start 89.965998 68.58) (end 67.31 68.58) (width 1.5) (layer B.Cu) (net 1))
 (segment (start 90.005998 68.54) (end 89.965998 68.58) (width 1.5) (layer B.Cu) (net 1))
 (segment (start 245.11 68.54) (end 90.005998 68.54) (width 1.5) (layer B.Cu) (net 1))
 (segment (start 58.37936 68.58) (end 57.15 69.80936) (width 1.5) (layer B.Cu) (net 1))
 (segment (start 67.31 68.58) (end 58.37936 68.58) (width 1.5) (layer B.Cu) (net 1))
 (segment (start 61.00064 73.66) (end 67.31 73.66) (width 1.5) (layer B.Cu) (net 1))
 (segment (start 207.367074 73.66) (end 245.11 73.66) (width 1.5) (layer B.Cu) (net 1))
 (segment (start 67.31 73.66) (end 207.367074 73.66) (width 1.5) (layer B.Cu) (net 1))
 (segment (start 245.11 73.66) (end 238.76 73.66) (width 1.5) (layer B.Cu) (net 1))
 (segment (start 240.03 68.58) (end 238.76 68.58) (width 1.5) (layer B.Cu) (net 1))
 (segment (start 58.46064 71.12) (end 57.15 69.80936) (width 1.5) (layer B.Cu) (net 1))
 (segment (start 236.22 71.12) (end 58.46064 71.12) (width 1.5) (layer B.Cu) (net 1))
 (segment (start 237.44936 69.80936) (end 237.49 69.85) (width 1.5) (layer B.Cu) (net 1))
 (segment (start 57.15 69.80936) (end 237.44936 69.80936) (width 1.5) (layer B.Cu) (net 1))
 (segment (start 237.49 69.85) (end 236.22 71.12) (width 1.5) (layer B.Cu) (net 1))
 (segment (start 238.76 68.58) (end 237.49 69.85) (width 1.5) (layer B.Cu) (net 1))
 (segment (start 237.49 72.39) (end 59.73064 72.39) (width 1.5) (layer B.Cu) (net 1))
 (segment (start 59.71032 72.36968) (end 61.00064 73.66) (width 1.5) (layer B.Cu) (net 1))
 (segment (start 57.15 69.80936) (end 59.71032 72.36968) (width 1.5) (layer B.Cu) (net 1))
 (segment (start 59.73064 72.39) (end 59.71032 72.36968) (width 1.5) (layer B.Cu) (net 1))
 (segment (start 238.76 73.66) (end 237.49 72.39) (width 1.5) (layer B.Cu) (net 1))
 (segment (start 237.49 72.39) (end 236.22 71.12) (width 1.5) (layer B.Cu) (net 1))
 (segment (start 57.19064 69.85) (end 57.15 69.80936) (width 1.5) (layer F.Cu) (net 1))
 (segment (start 237.49 69.85) (end 57.19064 69.85) (width 1.5) (layer F.Cu) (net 1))
 (segment (start 236.87532 72.36968) (end 237.1725 72.0725) (width 1.5) (layer F.Cu) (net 1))
 (segment (start 59.71032 72.36968) (end 236.87532 72.36968) (width 1.5) (layer F.Cu) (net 1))
 (segment (start 237.1725 72.0725) (end 236.22 71.12) (width 1.5) (layer F.Cu) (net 1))
 (segment (start 238.76 73.66) (end 237.1725 72.0725) (width 1.5) (layer F.Cu) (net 1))
 (segment (start 58.46064 76.2) (end 67.31 76.2) (width 1.5) (layer F.Cu) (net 2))
 (segment (start 57.15 74.88936) (end 58.46064 76.2) (width 1.5) (layer F.Cu) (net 2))
 (segment (start 245.07 76.2) (end 245.11 76.16) (width 1.5) (layer F.Cu) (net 2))
 (segment (start 67.31 76.2) (end 245.07 76.2) (width 1.5) (layer F.Cu) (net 2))
 (segment (start 58.46064 76.2) (end 67.31 76.2) (width 1.5) (layer B.Cu) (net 2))
 (segment (start 57.15 74.88936) (end 58.46064 76.2) (width 1.5) (layer B.Cu) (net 2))
 (segment (start 245.07 76.2) (end 245.11 76.16) (width 1.5) (layer B.Cu) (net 2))
 (segment (start 67.31 76.2) (end 245.07 76.2) (width 1.5) (layer B.Cu) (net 2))
 (segment (start 58.46064 66.04) (end 67.31 66.04) (width 1.5) (layer F.Cu) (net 3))
 (segment (start 57.15 64.72936) (end 58.46064 66.04) (width 1.5) (layer F.Cu) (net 3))
 (segment (start 67.31 66.04) (end 245.11 66.04) (width 1.5) (layer F.Cu) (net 3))
 (segment (start 204.345998 66.04) (end 184.15 66.04) (width 1.5) (layer B.Cu) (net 3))
 (segment (start 245.11 66.04) (end 204.345998 66.04) (width 1.5) (layer B.Cu) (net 3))
 (segment (start 58.46064 66.04) (end 57.15 64.72936) (width 1.5) (layer B.Cu) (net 3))
 (segment (start 184.15 66.04) (end 58.46064 66.04) (width 1.5) (layer B.Cu) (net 3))
 (segment (start 61.00064 63.5) (end 67.31 63.5) (width 1.5) (layer F.Cu) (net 4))
 (segment (start 57.15 59.64936) (end 61.00064 63.5) (width 1.5) (layer F.Cu) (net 4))
 (segment (start 67.31 63.5) (end 236.22 63.5) (width 1.5) (layer F.Cu) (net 4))
 (segment (start 240.03 63.5) (end 245.11 58.42) (width 1.5) (layer F.Cu) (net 4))
 (segment (start 236.22 63.5) (end 240.03 63.5) (width 1.5) (layer F.Cu) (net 4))
 (segment (start 240.03 63.5) (end 236.22 63.5) (width 1.5) (layer B.Cu) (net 4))
 (segment (start 245.11 58.42) (end 240.03 63.5) (width 1.5) (layer B.Cu) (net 4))
 (segment (start 61.00064 63.5) (end 67.31 63.5) (width 1.5) (layer B.Cu) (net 4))
 (segment (start 57.15 59.64936) (end 61.00064 63.5) (width 1.5) (layer B.Cu) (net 4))
 (segment (start 67.31 63.5) (end 236.22 63.5) (width 1.5) (layer B.Cu) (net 4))
 (segment (start 229.87 60.96) (end 67.31 60.96) (width 1.5) (layer F.Cu) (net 5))
 (segment (start 229.87 60.96) (end 67.31 60.96) (width 1.5) (layer B.Cu) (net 5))
 (segment (start 67.31 58.42) (end 229.87 58.42) (width 1.5) (layer F.Cu) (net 6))
 (segment (start 67.31 58.42) (end 229.87 58.42) (width 1.5) (layer B.Cu) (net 6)))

